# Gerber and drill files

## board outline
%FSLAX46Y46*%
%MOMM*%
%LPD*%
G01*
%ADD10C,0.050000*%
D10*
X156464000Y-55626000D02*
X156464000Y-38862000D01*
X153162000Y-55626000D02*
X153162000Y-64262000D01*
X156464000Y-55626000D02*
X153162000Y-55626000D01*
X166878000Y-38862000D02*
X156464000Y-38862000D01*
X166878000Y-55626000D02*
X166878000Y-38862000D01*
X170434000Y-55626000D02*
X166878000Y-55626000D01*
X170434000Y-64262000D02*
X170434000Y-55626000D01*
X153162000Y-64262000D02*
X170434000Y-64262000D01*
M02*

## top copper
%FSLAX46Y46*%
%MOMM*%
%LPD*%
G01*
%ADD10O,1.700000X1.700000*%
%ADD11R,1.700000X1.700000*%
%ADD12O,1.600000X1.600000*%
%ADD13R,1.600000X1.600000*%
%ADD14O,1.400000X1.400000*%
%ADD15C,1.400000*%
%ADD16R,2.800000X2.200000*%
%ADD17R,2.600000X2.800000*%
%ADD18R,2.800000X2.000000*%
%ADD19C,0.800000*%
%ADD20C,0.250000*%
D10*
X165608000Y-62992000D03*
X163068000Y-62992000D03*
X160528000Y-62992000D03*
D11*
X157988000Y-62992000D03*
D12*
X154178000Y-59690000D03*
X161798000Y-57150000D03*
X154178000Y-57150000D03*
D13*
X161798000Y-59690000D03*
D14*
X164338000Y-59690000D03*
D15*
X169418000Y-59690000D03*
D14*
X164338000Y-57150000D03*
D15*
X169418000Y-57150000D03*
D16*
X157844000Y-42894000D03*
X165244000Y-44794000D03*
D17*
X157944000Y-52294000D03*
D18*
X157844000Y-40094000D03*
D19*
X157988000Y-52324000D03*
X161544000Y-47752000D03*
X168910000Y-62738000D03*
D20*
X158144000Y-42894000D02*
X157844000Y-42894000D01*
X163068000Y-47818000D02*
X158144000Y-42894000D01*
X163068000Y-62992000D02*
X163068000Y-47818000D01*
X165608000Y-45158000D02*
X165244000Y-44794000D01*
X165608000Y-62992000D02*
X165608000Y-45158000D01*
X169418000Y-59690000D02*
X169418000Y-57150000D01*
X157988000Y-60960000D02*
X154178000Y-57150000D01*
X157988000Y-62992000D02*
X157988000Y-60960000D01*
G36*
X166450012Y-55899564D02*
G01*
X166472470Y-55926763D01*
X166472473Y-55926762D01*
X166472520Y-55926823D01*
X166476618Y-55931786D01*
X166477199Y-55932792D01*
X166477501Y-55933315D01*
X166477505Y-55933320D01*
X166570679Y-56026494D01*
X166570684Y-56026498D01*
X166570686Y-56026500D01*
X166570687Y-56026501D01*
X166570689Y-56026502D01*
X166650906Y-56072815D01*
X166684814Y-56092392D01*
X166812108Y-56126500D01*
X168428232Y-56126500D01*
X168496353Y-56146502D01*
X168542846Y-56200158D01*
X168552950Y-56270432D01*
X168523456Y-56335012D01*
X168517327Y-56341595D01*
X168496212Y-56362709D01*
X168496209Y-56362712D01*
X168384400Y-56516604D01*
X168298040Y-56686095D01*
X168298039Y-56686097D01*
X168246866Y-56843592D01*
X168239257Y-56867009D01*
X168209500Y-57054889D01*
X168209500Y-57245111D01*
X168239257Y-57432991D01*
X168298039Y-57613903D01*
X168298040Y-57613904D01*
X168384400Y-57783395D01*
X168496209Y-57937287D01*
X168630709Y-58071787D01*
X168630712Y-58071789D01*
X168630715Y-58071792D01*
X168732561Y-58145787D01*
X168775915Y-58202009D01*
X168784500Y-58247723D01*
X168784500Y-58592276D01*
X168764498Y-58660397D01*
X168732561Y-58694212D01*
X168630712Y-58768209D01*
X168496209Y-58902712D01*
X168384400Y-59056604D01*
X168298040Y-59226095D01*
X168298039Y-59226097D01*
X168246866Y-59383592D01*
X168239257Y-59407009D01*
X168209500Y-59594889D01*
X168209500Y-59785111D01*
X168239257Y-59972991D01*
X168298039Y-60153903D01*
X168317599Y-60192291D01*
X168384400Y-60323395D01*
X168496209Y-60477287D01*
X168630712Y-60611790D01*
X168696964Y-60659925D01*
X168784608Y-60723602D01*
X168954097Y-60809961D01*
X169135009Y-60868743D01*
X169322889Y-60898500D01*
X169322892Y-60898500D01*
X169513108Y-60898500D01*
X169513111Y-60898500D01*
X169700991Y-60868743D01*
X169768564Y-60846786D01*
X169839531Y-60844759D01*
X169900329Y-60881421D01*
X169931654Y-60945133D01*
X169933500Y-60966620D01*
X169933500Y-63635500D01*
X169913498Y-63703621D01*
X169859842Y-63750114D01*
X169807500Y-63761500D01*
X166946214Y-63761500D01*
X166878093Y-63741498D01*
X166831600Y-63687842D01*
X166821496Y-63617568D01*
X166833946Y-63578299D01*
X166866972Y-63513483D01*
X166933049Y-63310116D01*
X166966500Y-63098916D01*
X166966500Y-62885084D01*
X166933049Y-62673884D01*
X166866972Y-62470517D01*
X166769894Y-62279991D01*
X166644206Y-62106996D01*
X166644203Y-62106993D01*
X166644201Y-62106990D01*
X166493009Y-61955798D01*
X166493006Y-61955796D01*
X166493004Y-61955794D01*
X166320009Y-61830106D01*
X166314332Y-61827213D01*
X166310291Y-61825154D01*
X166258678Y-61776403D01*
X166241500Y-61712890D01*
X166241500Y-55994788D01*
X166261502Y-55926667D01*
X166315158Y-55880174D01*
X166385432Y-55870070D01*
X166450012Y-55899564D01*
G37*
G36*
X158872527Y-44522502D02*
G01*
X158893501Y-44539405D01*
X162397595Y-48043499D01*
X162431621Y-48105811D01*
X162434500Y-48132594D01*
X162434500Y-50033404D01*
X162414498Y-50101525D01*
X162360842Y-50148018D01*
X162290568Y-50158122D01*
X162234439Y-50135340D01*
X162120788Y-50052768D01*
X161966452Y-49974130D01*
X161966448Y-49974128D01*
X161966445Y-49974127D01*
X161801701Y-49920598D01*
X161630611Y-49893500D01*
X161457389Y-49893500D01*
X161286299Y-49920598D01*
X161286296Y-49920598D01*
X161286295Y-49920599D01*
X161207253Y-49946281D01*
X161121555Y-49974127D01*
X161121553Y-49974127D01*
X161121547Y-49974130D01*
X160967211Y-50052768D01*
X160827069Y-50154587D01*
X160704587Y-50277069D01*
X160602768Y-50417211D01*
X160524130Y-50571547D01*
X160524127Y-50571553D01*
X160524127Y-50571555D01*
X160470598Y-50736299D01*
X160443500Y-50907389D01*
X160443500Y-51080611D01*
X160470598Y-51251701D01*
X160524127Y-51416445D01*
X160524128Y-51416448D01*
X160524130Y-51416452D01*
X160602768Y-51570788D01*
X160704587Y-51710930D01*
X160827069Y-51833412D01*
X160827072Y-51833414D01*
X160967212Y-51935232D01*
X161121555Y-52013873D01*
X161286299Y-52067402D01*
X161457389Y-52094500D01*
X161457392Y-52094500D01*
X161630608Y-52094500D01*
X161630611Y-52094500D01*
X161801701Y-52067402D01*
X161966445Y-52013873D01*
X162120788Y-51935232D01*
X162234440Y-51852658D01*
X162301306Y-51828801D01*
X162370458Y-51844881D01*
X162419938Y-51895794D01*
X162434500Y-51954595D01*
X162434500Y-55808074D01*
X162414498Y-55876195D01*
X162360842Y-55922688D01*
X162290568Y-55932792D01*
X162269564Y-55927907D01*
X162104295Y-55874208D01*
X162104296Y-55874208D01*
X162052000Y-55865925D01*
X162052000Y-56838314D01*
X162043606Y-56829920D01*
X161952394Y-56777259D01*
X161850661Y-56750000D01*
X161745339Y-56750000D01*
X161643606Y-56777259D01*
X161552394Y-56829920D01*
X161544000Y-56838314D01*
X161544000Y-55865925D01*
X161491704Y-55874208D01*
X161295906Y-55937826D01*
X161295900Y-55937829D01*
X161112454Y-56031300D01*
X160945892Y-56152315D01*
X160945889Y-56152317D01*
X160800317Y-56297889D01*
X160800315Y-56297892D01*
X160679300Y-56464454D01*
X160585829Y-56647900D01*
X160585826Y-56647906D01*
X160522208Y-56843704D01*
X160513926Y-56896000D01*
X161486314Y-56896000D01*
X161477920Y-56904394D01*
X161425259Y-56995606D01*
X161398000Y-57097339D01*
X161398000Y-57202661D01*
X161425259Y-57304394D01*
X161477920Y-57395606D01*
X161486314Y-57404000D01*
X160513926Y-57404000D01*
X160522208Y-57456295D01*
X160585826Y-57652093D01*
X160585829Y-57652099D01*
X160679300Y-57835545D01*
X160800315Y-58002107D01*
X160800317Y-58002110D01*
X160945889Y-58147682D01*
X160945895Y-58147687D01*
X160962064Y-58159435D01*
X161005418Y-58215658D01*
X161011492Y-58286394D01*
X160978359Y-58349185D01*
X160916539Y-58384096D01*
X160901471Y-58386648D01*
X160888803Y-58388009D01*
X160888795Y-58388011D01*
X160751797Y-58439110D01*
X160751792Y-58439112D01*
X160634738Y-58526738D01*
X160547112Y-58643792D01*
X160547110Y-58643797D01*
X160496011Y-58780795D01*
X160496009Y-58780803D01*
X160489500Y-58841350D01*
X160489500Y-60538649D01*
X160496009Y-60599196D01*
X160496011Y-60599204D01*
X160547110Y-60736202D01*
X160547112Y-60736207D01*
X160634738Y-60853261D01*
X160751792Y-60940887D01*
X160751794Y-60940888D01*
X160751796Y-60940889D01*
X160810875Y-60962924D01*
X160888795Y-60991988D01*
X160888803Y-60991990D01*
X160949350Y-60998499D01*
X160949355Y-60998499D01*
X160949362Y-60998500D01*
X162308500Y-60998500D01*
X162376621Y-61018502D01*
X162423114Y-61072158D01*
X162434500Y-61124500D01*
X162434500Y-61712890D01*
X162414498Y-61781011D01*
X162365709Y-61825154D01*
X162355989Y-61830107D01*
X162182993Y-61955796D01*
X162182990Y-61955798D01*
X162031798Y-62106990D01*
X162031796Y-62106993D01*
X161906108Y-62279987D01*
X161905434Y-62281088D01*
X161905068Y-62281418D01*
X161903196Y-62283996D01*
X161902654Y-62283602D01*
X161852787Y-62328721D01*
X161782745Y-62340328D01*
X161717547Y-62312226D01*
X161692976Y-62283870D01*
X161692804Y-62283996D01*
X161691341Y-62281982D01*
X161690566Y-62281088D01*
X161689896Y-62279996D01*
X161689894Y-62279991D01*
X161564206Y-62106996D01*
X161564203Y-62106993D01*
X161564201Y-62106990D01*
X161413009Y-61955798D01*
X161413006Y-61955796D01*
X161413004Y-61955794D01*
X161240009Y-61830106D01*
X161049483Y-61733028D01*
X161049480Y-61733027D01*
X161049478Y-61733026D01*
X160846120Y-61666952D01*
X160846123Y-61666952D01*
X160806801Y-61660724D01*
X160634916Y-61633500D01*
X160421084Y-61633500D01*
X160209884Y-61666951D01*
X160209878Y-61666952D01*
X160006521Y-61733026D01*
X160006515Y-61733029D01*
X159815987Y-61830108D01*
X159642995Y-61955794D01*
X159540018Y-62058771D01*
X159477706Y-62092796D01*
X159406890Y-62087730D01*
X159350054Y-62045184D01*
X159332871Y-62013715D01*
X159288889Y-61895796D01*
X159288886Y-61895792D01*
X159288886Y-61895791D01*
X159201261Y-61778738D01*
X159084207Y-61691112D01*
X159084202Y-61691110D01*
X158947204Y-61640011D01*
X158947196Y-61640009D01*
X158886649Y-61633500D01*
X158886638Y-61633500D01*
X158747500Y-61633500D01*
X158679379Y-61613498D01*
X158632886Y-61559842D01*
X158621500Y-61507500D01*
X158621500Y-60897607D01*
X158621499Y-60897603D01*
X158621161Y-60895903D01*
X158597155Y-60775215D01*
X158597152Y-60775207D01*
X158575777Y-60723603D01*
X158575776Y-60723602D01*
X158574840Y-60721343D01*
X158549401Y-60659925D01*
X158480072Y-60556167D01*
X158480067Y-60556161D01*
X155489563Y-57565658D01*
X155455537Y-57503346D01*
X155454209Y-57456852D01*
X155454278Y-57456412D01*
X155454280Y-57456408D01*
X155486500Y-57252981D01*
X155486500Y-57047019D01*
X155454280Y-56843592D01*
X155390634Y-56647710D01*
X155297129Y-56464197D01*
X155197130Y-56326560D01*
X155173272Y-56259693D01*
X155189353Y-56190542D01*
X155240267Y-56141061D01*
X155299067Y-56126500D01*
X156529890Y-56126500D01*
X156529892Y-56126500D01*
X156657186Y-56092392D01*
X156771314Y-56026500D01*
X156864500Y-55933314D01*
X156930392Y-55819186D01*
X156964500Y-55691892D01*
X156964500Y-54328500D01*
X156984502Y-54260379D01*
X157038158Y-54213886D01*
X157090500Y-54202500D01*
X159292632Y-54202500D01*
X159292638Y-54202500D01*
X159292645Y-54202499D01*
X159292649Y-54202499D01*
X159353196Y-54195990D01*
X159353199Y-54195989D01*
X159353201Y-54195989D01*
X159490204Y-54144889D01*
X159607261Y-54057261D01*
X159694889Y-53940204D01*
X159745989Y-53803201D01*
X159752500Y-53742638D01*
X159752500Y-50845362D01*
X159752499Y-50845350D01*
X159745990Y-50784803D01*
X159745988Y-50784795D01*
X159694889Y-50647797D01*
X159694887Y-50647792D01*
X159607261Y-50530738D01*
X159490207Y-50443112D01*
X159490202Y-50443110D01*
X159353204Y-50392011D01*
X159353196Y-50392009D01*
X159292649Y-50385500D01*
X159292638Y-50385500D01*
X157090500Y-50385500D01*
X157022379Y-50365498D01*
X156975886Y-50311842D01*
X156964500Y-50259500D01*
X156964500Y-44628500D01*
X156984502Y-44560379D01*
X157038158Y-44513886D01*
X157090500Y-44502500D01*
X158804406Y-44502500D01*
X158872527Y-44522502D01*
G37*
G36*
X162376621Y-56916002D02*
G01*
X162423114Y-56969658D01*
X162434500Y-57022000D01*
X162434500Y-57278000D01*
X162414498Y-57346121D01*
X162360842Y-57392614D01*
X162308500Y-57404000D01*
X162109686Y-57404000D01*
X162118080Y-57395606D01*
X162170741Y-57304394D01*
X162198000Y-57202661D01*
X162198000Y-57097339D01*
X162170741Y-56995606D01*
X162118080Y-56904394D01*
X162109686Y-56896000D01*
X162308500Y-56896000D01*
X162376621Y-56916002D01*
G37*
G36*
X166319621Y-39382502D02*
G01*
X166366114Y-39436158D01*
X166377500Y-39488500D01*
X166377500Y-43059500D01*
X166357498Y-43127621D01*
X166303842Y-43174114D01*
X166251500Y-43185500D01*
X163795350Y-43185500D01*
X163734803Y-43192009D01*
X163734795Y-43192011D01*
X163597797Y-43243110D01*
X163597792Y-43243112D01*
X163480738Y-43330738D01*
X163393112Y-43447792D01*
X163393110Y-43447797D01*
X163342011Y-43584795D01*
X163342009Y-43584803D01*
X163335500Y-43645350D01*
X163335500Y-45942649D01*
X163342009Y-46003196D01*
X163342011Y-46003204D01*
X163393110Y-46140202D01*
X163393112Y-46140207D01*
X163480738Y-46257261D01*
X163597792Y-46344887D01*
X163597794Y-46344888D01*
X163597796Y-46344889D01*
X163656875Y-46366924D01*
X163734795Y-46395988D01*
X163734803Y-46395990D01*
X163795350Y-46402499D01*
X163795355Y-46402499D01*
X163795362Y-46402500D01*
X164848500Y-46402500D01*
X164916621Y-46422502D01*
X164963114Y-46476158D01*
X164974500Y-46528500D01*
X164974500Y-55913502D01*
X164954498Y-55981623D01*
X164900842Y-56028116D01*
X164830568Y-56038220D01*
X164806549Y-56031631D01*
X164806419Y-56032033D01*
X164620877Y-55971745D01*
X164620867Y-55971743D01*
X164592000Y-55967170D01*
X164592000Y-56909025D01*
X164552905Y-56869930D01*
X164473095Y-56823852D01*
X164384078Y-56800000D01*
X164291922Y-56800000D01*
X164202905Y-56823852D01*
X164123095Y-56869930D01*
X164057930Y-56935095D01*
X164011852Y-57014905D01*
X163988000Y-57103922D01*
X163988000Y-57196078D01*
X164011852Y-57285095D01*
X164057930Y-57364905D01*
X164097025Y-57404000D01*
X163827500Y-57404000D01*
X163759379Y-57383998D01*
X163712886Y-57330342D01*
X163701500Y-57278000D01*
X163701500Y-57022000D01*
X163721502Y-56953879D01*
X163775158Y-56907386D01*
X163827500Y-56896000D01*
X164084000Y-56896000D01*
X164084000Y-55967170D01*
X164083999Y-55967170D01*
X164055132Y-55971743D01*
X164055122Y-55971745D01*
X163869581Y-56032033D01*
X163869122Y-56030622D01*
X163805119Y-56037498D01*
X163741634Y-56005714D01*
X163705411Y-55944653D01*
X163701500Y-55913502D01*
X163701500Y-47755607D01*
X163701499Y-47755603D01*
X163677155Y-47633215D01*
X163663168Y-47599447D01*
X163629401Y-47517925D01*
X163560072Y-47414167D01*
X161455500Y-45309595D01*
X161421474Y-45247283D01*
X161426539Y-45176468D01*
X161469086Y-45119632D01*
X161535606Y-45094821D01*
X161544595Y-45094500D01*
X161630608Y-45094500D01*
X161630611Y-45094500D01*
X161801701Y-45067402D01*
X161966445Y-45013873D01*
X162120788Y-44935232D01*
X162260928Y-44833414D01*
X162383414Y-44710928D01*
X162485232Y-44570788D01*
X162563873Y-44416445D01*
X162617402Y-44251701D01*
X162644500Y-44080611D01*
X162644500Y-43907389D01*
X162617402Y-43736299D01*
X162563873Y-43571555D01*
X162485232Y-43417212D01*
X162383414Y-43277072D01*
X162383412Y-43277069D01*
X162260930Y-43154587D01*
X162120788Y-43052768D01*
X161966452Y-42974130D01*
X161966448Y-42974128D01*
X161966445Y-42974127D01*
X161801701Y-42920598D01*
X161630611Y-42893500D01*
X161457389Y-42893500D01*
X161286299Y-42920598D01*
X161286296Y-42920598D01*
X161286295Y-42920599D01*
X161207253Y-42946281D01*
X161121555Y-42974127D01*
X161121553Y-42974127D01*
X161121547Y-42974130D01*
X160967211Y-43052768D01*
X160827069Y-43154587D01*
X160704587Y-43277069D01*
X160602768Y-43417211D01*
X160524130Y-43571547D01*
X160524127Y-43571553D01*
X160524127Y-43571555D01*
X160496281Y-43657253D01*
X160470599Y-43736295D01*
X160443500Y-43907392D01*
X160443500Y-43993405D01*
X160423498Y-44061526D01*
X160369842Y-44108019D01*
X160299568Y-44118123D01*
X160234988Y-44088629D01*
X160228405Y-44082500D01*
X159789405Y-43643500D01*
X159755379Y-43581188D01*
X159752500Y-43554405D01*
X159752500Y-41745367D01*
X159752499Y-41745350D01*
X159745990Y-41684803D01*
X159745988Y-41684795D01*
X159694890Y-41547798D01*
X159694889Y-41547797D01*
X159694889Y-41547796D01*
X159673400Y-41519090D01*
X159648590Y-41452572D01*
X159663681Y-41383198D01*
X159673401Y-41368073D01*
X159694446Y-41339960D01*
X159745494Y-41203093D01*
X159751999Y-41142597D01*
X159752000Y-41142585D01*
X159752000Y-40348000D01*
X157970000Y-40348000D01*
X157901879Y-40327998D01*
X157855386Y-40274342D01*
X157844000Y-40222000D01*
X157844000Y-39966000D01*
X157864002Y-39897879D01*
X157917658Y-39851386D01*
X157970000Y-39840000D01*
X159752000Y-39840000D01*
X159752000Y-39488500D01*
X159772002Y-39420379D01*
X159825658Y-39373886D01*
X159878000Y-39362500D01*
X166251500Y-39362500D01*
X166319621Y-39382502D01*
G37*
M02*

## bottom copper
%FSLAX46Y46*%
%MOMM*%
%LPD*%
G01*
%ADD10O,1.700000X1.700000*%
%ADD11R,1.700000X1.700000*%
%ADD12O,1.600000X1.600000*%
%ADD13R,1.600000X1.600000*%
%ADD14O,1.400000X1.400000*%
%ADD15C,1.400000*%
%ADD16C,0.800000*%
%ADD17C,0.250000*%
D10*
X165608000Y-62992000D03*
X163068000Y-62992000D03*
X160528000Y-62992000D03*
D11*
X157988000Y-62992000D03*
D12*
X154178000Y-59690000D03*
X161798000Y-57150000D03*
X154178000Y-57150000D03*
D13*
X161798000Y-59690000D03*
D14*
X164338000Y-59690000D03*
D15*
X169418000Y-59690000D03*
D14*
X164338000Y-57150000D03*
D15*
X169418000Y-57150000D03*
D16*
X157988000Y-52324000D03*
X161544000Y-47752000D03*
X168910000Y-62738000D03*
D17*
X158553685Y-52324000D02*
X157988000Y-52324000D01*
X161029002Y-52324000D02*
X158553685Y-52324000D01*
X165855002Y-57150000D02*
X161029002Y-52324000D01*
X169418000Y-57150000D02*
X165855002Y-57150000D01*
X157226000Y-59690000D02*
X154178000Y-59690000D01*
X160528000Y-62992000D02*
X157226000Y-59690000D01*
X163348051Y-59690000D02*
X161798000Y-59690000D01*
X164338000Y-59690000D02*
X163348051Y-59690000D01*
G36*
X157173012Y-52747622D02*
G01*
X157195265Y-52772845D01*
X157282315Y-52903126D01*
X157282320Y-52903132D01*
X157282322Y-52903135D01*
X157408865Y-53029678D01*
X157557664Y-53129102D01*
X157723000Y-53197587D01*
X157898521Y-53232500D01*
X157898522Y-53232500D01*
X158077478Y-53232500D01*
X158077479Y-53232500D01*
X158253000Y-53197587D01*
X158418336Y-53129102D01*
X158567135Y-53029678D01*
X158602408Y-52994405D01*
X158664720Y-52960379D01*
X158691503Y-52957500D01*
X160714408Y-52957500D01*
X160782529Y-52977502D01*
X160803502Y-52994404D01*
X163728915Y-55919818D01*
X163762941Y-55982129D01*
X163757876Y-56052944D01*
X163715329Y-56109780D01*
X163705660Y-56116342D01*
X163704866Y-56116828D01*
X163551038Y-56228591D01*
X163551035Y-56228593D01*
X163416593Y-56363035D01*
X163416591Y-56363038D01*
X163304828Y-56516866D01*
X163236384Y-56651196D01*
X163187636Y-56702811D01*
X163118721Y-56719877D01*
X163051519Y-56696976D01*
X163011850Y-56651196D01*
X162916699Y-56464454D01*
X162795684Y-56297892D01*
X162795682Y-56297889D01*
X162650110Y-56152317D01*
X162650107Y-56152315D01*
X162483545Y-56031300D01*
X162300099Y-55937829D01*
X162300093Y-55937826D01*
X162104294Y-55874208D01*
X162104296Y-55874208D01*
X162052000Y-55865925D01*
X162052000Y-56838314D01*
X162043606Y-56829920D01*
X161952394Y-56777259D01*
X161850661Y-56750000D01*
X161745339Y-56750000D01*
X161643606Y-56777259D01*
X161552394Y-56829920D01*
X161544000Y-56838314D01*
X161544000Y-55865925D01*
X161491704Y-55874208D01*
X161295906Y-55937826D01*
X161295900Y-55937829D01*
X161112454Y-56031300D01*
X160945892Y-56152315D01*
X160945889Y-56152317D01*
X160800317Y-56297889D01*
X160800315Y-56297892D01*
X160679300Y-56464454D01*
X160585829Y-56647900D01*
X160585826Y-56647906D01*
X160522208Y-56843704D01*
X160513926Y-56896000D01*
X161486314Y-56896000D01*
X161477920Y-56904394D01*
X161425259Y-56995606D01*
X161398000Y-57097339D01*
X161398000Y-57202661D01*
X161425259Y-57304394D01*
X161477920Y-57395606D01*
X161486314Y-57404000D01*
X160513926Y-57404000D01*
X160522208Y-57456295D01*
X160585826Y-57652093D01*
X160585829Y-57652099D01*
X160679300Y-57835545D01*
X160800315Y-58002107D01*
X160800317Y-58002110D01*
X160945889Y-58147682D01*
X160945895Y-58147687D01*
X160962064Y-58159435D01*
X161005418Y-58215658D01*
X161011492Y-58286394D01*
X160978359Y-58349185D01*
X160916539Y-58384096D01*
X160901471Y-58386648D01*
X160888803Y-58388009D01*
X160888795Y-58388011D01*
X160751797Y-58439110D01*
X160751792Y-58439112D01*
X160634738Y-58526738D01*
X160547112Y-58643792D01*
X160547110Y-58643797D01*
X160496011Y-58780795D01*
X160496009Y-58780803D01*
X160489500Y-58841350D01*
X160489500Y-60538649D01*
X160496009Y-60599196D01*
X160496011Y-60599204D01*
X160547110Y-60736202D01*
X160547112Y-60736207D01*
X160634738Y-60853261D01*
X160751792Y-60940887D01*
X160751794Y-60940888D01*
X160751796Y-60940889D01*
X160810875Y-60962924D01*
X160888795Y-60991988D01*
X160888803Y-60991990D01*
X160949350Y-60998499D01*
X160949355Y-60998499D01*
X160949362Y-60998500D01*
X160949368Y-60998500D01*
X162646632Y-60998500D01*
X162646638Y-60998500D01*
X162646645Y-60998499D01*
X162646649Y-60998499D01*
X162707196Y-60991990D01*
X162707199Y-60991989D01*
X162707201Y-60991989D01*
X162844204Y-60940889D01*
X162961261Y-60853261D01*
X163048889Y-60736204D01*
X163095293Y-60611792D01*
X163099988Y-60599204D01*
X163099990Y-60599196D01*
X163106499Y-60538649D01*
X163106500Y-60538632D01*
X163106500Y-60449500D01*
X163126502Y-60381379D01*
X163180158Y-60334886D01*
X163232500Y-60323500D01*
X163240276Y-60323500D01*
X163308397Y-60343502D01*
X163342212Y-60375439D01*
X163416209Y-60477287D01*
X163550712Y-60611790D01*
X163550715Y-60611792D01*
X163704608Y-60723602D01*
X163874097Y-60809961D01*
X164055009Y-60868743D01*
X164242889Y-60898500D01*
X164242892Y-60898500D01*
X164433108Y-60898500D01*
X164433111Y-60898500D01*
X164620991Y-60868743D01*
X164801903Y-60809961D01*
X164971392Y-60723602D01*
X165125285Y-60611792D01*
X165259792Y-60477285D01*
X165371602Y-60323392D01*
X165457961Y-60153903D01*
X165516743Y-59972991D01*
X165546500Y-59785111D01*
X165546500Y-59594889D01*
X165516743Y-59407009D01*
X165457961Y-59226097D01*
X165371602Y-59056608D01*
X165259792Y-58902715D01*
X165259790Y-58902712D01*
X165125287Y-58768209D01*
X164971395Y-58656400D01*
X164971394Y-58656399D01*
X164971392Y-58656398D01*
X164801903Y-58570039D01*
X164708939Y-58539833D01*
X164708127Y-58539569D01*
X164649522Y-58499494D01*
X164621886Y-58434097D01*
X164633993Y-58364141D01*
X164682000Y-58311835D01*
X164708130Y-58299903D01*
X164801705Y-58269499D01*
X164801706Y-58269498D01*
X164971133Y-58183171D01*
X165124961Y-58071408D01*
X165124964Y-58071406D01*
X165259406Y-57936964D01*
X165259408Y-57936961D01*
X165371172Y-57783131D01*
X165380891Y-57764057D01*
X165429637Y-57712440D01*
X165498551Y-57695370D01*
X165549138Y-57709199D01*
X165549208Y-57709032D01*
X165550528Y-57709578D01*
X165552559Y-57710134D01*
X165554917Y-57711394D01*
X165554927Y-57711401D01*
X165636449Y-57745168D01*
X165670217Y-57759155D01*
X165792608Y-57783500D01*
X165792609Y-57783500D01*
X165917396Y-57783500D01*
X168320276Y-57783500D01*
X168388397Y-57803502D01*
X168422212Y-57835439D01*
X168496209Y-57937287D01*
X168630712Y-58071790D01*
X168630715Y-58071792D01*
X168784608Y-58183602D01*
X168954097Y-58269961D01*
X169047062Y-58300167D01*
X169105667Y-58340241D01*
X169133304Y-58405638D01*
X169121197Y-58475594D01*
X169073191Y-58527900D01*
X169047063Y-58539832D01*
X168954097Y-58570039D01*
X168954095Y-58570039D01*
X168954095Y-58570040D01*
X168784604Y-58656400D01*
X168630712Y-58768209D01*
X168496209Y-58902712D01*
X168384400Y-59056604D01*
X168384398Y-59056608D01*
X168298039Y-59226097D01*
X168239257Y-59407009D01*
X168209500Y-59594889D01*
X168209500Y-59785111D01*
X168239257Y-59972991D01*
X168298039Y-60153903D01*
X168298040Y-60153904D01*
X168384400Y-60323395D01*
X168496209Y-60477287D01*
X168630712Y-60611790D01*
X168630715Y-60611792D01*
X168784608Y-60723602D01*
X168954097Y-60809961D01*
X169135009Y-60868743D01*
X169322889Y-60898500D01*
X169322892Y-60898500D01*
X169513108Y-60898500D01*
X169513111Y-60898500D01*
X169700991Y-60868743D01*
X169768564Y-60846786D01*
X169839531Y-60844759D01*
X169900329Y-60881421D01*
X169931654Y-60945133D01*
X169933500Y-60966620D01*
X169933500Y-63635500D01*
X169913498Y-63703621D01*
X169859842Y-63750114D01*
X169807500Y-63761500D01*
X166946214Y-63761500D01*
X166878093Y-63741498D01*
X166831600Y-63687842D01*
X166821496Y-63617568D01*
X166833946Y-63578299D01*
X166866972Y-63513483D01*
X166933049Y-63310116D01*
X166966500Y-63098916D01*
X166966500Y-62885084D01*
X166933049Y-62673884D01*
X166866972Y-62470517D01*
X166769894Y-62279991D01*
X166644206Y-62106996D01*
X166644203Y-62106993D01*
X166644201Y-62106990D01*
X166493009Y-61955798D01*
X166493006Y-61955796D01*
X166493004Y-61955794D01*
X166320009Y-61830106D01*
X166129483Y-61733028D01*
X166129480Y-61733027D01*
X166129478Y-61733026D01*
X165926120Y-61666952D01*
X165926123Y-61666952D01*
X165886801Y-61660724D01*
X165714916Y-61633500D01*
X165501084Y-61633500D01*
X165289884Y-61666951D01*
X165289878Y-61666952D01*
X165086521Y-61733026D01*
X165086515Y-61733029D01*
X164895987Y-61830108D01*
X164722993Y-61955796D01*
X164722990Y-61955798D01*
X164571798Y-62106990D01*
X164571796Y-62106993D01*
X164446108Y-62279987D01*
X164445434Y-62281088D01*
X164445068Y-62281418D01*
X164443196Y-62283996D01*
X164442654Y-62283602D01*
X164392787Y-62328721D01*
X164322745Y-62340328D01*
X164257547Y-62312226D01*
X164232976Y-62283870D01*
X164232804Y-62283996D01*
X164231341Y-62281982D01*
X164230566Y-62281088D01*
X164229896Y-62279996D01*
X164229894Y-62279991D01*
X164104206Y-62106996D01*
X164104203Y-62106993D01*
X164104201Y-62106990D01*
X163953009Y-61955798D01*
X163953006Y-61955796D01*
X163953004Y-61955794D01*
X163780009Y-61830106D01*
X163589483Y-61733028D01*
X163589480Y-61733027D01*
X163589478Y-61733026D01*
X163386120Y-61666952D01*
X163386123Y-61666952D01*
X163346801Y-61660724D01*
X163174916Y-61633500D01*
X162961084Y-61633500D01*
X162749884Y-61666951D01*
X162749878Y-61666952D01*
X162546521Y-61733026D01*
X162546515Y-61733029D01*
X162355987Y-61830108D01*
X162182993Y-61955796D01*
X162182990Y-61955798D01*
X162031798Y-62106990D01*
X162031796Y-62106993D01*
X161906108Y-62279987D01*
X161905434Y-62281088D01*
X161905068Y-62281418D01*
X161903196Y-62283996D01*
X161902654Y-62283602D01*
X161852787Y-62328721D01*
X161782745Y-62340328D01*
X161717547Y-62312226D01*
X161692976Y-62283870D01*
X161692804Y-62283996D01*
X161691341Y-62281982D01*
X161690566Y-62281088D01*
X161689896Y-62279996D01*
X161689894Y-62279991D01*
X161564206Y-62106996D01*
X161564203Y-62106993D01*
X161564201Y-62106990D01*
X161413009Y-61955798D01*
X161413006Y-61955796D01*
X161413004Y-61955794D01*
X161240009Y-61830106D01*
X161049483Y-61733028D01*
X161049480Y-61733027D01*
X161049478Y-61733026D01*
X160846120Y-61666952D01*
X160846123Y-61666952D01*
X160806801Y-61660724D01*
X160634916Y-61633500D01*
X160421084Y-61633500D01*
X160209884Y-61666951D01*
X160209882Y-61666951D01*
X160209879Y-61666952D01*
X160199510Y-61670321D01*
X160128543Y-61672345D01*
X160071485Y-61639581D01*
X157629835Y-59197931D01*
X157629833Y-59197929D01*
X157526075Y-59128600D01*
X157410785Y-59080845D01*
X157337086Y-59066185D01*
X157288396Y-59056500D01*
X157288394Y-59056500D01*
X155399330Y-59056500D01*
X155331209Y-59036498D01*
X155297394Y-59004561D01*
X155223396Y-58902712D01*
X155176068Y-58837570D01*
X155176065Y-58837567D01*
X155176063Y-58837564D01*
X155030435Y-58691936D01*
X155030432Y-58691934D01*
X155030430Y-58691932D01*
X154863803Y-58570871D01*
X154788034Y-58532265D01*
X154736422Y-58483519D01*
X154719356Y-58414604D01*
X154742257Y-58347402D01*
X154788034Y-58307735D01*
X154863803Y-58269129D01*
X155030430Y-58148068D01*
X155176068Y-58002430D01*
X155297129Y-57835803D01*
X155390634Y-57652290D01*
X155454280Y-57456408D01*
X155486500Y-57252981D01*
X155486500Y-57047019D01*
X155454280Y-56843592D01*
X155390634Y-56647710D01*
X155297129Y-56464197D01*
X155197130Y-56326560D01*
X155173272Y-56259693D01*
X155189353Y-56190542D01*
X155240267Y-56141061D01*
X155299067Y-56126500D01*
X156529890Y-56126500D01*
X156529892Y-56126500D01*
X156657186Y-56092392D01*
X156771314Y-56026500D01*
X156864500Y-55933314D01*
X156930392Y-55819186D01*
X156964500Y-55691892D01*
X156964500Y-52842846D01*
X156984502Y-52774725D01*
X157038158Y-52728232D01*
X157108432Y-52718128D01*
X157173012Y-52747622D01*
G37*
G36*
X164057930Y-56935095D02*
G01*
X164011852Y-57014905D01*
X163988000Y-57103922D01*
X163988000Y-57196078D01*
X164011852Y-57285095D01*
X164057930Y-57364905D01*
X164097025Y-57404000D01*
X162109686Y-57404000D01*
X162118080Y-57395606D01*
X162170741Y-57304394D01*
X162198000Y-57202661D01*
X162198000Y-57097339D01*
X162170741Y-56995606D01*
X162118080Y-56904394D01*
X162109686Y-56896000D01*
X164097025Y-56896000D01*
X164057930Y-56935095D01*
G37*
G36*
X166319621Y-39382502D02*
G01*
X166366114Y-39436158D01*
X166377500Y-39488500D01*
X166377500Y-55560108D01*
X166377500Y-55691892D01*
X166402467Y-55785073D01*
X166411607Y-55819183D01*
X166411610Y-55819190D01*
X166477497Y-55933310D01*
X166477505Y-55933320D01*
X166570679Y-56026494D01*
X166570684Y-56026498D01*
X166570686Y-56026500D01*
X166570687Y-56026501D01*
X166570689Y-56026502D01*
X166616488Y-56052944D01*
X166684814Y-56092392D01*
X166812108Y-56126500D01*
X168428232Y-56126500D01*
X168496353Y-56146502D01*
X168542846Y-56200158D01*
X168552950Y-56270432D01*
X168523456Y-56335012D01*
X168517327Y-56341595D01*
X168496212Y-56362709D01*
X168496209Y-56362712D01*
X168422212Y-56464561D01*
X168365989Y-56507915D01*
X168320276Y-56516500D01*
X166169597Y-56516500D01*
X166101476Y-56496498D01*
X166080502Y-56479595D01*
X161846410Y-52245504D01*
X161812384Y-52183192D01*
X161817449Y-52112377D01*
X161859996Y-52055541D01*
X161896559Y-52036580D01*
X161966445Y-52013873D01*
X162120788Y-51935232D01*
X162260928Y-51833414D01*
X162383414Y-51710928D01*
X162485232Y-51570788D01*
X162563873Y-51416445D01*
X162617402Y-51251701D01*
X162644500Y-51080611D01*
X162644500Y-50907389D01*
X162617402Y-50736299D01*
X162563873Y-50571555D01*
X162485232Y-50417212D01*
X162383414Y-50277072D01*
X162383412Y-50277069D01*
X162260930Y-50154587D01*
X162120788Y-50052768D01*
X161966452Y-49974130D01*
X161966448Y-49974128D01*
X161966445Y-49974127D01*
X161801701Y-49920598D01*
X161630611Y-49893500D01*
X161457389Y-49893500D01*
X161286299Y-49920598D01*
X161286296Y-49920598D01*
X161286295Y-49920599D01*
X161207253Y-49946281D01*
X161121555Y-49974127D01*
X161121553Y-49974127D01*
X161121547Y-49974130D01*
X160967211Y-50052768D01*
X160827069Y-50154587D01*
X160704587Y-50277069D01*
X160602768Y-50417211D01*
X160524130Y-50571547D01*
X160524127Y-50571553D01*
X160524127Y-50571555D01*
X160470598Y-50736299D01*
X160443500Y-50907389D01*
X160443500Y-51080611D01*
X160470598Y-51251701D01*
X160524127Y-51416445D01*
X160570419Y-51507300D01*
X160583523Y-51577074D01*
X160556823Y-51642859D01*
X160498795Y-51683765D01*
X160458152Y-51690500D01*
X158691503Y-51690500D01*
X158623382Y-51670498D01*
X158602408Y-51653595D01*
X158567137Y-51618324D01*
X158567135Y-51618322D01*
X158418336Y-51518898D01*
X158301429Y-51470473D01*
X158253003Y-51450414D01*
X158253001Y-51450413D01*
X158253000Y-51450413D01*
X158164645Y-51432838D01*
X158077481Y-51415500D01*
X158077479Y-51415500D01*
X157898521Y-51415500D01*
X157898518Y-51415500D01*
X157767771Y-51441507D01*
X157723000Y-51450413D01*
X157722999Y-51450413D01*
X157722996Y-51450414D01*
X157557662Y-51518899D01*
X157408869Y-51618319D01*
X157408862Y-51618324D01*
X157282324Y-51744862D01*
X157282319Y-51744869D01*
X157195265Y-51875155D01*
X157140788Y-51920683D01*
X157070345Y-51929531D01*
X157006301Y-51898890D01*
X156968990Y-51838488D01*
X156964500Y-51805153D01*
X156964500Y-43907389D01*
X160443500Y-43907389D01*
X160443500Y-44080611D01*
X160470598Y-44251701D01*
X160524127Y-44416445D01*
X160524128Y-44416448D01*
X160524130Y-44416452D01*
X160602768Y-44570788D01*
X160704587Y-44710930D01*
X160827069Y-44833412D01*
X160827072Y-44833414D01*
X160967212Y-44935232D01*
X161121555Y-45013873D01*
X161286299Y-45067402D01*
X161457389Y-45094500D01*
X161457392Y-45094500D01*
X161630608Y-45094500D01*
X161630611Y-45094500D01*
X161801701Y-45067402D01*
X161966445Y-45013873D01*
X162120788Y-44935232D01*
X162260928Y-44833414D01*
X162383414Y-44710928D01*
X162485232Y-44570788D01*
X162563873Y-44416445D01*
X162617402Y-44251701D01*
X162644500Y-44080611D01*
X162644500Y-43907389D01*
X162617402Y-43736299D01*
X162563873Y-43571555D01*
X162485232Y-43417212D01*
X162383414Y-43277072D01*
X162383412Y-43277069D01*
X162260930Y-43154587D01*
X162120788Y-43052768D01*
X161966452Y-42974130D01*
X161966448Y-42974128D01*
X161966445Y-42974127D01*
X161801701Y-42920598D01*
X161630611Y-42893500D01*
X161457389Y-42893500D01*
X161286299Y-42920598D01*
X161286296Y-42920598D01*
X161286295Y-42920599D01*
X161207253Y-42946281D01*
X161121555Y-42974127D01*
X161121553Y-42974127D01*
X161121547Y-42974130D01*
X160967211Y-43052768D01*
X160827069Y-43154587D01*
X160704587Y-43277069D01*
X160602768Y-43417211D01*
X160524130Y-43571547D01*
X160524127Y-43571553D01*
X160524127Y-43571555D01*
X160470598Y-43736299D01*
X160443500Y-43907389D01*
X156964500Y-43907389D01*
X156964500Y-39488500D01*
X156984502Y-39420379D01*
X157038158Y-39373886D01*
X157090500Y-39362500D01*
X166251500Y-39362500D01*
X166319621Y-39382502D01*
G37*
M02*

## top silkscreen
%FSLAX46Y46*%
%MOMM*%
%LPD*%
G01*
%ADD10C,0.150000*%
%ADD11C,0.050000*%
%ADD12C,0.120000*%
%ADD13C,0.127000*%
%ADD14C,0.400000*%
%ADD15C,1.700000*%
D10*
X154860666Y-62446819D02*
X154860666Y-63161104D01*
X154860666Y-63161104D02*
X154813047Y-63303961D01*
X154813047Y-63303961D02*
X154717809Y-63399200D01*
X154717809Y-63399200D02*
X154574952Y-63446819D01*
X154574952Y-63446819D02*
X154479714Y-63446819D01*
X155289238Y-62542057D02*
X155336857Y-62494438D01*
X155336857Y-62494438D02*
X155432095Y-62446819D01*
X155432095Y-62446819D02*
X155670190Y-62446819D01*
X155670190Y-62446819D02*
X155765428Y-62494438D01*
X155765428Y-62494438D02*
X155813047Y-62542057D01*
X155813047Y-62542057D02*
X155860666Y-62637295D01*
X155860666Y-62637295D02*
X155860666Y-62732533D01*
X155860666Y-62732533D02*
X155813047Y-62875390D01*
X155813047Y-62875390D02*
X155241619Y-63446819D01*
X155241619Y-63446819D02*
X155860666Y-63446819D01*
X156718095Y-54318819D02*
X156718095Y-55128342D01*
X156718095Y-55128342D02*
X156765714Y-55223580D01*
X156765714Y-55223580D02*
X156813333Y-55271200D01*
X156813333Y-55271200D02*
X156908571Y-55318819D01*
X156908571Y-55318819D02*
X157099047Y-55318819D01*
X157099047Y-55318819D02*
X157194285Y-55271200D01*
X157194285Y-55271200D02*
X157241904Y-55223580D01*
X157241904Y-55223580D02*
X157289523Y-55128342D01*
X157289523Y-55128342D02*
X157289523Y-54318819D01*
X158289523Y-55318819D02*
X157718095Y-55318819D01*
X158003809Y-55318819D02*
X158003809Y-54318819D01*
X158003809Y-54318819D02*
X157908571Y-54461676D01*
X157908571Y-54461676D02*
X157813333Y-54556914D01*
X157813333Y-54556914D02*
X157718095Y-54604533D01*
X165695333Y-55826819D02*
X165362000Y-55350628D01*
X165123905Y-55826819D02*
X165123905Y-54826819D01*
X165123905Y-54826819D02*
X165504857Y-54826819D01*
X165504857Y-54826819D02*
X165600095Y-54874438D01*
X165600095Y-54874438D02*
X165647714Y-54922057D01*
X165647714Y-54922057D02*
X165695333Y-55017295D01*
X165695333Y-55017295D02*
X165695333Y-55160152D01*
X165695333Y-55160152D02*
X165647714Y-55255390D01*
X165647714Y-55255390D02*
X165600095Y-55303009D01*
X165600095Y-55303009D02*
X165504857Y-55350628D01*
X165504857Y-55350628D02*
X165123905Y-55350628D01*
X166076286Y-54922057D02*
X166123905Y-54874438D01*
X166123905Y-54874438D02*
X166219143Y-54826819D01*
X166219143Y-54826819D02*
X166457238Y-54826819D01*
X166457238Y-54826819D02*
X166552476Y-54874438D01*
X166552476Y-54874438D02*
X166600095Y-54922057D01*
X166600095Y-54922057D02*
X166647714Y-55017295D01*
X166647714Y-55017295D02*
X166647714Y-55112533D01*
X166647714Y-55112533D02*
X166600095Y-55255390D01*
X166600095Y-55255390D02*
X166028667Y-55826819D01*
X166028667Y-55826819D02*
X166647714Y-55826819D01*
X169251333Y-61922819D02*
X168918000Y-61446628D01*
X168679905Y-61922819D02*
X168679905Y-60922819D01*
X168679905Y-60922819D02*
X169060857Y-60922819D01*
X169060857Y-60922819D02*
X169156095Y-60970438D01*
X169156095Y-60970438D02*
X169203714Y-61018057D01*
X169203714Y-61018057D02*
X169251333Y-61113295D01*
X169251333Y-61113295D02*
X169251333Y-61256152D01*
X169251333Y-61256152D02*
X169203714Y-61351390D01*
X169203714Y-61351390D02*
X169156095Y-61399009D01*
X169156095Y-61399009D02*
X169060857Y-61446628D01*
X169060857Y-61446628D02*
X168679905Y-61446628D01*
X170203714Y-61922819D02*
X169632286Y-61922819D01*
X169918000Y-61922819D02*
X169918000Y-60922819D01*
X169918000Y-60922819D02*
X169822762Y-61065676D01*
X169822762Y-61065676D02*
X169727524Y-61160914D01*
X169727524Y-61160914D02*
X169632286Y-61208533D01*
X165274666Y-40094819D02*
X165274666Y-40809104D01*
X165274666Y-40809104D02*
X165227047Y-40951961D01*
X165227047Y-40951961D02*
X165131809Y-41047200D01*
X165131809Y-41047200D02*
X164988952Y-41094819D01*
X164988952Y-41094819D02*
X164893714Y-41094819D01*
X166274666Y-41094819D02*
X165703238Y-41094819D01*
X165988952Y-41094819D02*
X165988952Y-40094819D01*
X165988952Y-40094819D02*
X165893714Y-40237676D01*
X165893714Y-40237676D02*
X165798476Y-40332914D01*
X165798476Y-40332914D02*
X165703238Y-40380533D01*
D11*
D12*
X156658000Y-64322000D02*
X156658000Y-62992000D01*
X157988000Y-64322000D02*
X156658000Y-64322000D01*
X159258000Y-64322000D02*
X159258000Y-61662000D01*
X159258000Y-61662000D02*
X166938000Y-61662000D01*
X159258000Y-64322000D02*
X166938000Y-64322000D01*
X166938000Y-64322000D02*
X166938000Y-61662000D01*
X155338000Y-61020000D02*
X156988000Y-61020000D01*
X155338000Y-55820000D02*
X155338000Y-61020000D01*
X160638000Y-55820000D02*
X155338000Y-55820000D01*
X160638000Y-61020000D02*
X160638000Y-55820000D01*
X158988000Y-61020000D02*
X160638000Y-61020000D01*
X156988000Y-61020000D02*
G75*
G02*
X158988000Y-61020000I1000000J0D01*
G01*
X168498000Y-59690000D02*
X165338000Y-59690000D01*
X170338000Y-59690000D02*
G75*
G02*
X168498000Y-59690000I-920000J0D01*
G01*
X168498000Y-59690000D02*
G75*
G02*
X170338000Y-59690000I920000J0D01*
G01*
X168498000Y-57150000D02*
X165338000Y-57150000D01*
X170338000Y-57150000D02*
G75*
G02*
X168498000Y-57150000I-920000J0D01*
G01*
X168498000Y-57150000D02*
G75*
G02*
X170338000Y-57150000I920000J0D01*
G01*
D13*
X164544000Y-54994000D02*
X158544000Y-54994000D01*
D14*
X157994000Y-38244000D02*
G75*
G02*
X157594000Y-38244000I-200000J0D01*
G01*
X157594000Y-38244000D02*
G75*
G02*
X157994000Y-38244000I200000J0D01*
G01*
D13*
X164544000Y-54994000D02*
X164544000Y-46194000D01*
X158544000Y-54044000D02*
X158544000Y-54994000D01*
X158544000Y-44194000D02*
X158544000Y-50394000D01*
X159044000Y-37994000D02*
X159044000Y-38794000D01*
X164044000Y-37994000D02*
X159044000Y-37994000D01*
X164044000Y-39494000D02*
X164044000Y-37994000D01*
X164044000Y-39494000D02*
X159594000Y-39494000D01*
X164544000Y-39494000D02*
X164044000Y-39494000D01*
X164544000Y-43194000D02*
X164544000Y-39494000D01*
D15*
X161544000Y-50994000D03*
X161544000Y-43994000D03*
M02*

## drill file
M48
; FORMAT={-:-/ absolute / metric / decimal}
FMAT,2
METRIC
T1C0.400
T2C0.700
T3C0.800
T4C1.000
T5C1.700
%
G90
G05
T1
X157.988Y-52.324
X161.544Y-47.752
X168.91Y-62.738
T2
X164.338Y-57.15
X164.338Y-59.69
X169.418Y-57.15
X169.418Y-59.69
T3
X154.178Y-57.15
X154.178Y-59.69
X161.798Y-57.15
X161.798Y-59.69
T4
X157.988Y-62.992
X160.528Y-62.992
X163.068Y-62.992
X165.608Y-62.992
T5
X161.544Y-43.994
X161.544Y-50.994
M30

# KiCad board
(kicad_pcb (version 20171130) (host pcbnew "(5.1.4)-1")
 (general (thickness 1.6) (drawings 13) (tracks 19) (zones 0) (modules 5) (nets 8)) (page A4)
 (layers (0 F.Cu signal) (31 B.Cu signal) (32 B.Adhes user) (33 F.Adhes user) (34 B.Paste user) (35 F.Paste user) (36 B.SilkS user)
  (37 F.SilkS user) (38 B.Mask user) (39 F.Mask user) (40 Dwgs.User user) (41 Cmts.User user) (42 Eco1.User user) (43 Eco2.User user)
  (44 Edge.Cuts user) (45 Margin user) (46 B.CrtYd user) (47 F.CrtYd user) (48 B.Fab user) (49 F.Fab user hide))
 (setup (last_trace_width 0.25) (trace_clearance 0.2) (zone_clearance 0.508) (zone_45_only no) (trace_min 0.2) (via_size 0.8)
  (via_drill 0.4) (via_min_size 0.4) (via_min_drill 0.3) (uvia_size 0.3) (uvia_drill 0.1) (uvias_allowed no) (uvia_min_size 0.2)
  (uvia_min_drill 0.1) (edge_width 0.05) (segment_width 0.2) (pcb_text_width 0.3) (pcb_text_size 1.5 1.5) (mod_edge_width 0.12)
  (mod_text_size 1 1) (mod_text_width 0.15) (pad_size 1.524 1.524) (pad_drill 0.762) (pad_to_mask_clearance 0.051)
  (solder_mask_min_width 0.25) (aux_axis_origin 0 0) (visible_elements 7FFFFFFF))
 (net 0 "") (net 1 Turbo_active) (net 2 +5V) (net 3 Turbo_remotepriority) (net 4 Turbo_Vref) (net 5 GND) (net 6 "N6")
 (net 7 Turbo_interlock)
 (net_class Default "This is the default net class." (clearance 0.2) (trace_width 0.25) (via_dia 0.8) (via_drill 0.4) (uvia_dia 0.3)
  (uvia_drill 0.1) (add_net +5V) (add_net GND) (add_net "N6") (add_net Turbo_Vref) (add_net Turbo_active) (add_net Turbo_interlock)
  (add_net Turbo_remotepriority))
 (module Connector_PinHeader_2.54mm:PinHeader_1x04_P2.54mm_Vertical (layer F.Cu) (at 157.988 62.992 90)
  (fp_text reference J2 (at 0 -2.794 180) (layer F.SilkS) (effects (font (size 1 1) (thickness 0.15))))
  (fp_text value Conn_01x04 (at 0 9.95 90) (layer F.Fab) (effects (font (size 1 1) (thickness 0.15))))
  (fp_line (start -1.33 -1.33) (end 0 -1.33) (layer F.SilkS) (width 0.12))
  (fp_line (start -1.33 0) (end -1.33 -1.33) (layer F.SilkS) (width 0.12))
  (fp_line (start -1.33 1.27) (end 1.33 1.27) (layer F.SilkS) (width 0.12))
  (fp_line (start 1.33 1.27) (end 1.33 8.95) (layer F.SilkS) (width 0.12))
  (fp_line (start -1.33 1.27) (end -1.33 8.95) (layer F.SilkS) (width 0.12))
  (fp_line (start -1.33 8.95) (end 1.33 8.95) (layer F.SilkS) (width 0.12))
  (pad 4 thru_hole oval (at 0 7.62 90) (size 1.7 1.7) (drill 1) (layers *.Cu *.Mask) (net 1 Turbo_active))
  (pad 3 thru_hole oval (at 0 5.08 90) (size 1.7 1.7) (drill 1) (layers *.Cu *.Mask) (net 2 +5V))
  (pad 2 thru_hole oval (at 0 2.54 90) (size 1.7 1.7) (drill 1) (layers *.Cu *.Mask) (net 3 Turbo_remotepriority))
  (pad 1 thru_hole rect (at 0 0 90) (size 1.7 1.7) (drill 1) (layers *.Cu *.Mask) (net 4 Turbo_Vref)))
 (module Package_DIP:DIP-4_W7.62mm (layer F.Cu) (at 161.798 59.69 180)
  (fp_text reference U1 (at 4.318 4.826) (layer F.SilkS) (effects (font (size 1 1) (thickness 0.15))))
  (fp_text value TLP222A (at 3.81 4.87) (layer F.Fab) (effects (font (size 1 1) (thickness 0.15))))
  (fp_line (start 6.46 -1.33) (end 4.81 -1.33) (layer F.SilkS) (width 0.12))
  (fp_line (start 6.46 3.87) (end 6.46 -1.33) (layer F.SilkS) (width 0.12))
  (fp_line (start 1.16 3.87) (end 6.46 3.87) (layer F.SilkS) (width 0.12))
  (fp_line (start 1.16 -1.33) (end 1.16 3.87) (layer F.SilkS) (width 0.12))
  (fp_line (start 2.81 -1.33) (end 1.16 -1.33) (layer F.SilkS) (width 0.12))
  (fp_arc (start 3.81 -1.33) (end 2.81 -1.33) (angle -180) (layer F.SilkS) (width 0.12))
  (pad 4 thru_hole oval (at 7.62 0 180) (size 1.6 1.6) (drill 0.8) (layers *.Cu *.Mask) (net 3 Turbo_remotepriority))
  (pad 2 thru_hole oval (at 0 2.54 180) (size 1.6 1.6) (drill 0.8) (layers *.Cu *.Mask) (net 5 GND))
  (pad 3 thru_hole oval (at 7.62 2.54 180) (size 1.6 1.6) (drill 0.8) (layers *.Cu *.Mask) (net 4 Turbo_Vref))
  (pad 1 thru_hole rect (at 0 0 180) (size 1.6 1.6) (drill 0.8) (layers *.Cu *.Mask) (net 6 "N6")))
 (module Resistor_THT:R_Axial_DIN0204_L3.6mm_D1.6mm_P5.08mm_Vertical (layer F.Cu) (at 169.418 59.69 180)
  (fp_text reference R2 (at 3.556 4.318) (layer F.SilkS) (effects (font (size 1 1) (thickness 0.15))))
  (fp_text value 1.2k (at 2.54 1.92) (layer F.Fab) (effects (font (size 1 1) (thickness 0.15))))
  (fp_line (start 0.92 0) (end 4.08 0) (layer F.SilkS) (width 0.12))
  (fp_circle (center 0 0) (end 0.92 0) (layer F.SilkS) (width 0.12))
  (pad 2 thru_hole oval (at 5.08 0 180) (size 1.4 1.4) (drill 0.7) (layers *.Cu *.Mask) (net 6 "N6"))
  (pad 1 thru_hole circle (at 0 0 180) (size 1.4 1.4) (drill 0.7) (layers *.Cu *.Mask) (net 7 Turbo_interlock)))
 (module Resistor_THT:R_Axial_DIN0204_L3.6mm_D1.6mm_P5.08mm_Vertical (layer F.Cu) (at 169.418 57.15 180)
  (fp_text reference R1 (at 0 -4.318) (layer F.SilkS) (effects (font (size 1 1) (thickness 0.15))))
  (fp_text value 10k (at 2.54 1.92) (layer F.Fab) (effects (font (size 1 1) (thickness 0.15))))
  (fp_line (start 0.92 0) (end 4.08 0) (layer F.SilkS) (width 0.12))
  (fp_circle (center 0 0) (end 0.92 0) (layer F.SilkS) (width 0.12))
  (pad 2 thru_hole oval (at 5.08 0 180) (size 1.4 1.4) (drill 0.7) (layers *.Cu *.Mask) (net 5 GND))
  (pad 1 thru_hole circle (at 0 0 180) (size 1.4 1.4) (drill 0.7) (layers *.Cu *.Mask) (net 7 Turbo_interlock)))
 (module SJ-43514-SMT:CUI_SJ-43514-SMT (layer F.Cu) (at 161.544 47.244 270)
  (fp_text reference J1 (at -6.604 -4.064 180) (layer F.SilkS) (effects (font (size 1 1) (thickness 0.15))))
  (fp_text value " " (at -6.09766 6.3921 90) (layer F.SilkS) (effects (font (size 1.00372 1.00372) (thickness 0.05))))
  (fp_line (start 7.75 -3) (end 7.75 3) (layer F.SilkS) (width 0.127))
  (fp_circle (center -9 3.75) (end -8.8 3.75) (layer F.SilkS) (width 0.4))
  (fp_line (start 7.75 -3) (end -1.05 -3) (layer F.SilkS) (width 0.127))
  (fp_line (start 6.8 3) (end 7.75 3) (layer F.SilkS) (width 0.127))
  (fp_line (start -3.05 3) (end 3.15 3) (layer F.SilkS) (width 0.127))
  (fp_line (start -9.25 2.5) (end -8.45 2.5) (layer F.SilkS) (width 0.127))
  (fp_line (start -9.25 -2.5) (end -9.25 2.5) (layer F.SilkS) (width 0.127))
  (fp_line (start -7.75 -2.5) (end -9.25 -2.5) (layer F.SilkS) (width 0.127))
  (fp_line (start -7.75 -2.5) (end -7.75 1.95) (layer F.SilkS) (width 0.127))
  (fp_line (start -7.75 -3) (end -7.75 -2.5) (layer F.SilkS) (width 0.127))
  (fp_line (start -4.05 -3) (end -7.75 -3) (layer F.SilkS) (width 0.127))
  (pad Hole np_thru_hole circle (at 3.75 0 270) (size 1.7 1.7) (drill 1.7) (layers *.Cu *.Mask F.SilkS))
  (pad Hole np_thru_hole circle (at -3.25 0 270) (size 1.7 1.7) (drill 1.7) (layers *.Cu *.Mask F.SilkS))
  (pad 4 smd rect (at -4.35 3.7 90) (size 2.2 2.8) (layers F.Cu F.Paste F.Mask) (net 2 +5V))
  (pad 3 smd rect (at -2.45 -3.7 90) (size 2.2 2.8) (layers F.Cu F.Paste F.Mask) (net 1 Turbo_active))
  (pad 2 smd rect (at 5.05 3.6 90) (size 2.8 2.6) (layers F.Cu F.Paste F.Mask) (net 7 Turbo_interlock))
  (pad 1 smd rect (at -7.15 3.7 90) (size 2 2.8) (layers F.Cu F.Paste F.Mask) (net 5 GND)))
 (gr_line (start 156.464 55.626) (end 156.464 38.862) (layer Edge.Cuts) (width 0.05))
 (gr_line (start 153.162 55.626) (end 153.162 64.262) (layer Edge.Cuts) (width 0.05))
 (gr_line (start 156.464 55.626) (end 153.162 55.626) (layer Edge.Cuts) (width 0.05))
 (gr_line (start 166.878 38.862) (end 156.464 38.862) (layer Edge.Cuts) (width 0.05))
 (gr_line (start 166.878 55.626) (end 166.878 38.862) (layer Edge.Cuts) (width 0.05))
 (gr_line (start 170.434 55.626) (end 166.878 55.626) (layer Edge.Cuts) (width 0.05))
 (gr_line (start 170.434 64.262) (end 170.434 55.626) (layer Edge.Cuts) (width 0.05))
 (gr_line (start 153.162 64.262) (end 170.434 64.262) (layer Edge.Cuts) (width 0.05))
 (segment (start 158.144 42.894) (end 157.844 42.894) (width 0.25) (layer F.Cu) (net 2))
 (segment (start 163.068 47.818) (end 158.144 42.894) (width 0.25) (layer F.Cu) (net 2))
 (segment (start 163.068 62.992) (end 163.068 47.818) (width 0.25) (layer F.Cu) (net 2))
 (segment (start 165.608 45.158) (end 165.244 44.794) (width 0.25) (layer F.Cu) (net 1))
 (segment (start 165.608 62.992) (end 165.608 45.158) (width 0.25) (layer F.Cu) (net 1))
 (via (at 157.988 52.324) (size 0.8) (drill 0.4) (layers F.Cu B.Cu) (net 7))
 (segment (start 169.418 59.69) (end 169.418 57.15) (width 0.25) (layer F.Cu) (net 7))
 (segment (start 158.553685 52.324) (end 157.988 52.324) (width 0.25) (layer B.Cu) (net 7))
 (segment (start 161.029002 52.324) (end 158.553685 52.324) (width 0.25) (layer B.Cu) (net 7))
 (segment (start 165.855002 57.15) (end 161.029002 52.324) (width 0.25) (layer B.Cu) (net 7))
 (segment (start 169.418 57.15) (end 165.855002 57.15) (width 0.25) (layer B.Cu) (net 7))
 (via (at 161.544 47.752) (size 0.8) (drill 0.4) (layers F.Cu B.Cu) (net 5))
 (via (at 168.91 62.738) (size 0.8) (drill 0.4) (layers F.Cu B.Cu) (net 5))
 (segment (start 157.226 59.69) (end 154.178 59.69) (width 0.25) (layer B.Cu) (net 3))
 (segment (start 160.528 62.992) (end 157.226 59.69) (width 0.25) (layer B.Cu) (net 3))
 (segment (start 157.988 60.96) (end 154.178 57.15) (width 0.25) (layer F.Cu) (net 4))
 (segment (start 157.988 62.992) (end 157.988 60.96) (width 0.25) (layer F.Cu) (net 4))
 (segment (start 163.348051 59.69) (end 161.798 59.69) (width 0.25) (layer B.Cu) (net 6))
 (segment (start 164.338 59.69) (end 163.348051 59.69) (width 0.25) (layer B.Cu) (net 6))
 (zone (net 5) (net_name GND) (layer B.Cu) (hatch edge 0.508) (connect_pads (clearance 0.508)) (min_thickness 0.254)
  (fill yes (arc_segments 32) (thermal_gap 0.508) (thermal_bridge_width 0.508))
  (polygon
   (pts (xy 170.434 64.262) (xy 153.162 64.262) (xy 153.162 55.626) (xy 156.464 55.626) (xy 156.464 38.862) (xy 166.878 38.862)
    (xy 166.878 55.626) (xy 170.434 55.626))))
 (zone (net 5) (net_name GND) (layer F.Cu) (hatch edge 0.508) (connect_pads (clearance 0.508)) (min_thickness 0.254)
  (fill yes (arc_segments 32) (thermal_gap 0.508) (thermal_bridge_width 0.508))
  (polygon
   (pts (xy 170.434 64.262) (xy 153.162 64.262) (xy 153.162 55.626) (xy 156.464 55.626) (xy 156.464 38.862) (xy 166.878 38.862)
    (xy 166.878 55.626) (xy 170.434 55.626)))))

